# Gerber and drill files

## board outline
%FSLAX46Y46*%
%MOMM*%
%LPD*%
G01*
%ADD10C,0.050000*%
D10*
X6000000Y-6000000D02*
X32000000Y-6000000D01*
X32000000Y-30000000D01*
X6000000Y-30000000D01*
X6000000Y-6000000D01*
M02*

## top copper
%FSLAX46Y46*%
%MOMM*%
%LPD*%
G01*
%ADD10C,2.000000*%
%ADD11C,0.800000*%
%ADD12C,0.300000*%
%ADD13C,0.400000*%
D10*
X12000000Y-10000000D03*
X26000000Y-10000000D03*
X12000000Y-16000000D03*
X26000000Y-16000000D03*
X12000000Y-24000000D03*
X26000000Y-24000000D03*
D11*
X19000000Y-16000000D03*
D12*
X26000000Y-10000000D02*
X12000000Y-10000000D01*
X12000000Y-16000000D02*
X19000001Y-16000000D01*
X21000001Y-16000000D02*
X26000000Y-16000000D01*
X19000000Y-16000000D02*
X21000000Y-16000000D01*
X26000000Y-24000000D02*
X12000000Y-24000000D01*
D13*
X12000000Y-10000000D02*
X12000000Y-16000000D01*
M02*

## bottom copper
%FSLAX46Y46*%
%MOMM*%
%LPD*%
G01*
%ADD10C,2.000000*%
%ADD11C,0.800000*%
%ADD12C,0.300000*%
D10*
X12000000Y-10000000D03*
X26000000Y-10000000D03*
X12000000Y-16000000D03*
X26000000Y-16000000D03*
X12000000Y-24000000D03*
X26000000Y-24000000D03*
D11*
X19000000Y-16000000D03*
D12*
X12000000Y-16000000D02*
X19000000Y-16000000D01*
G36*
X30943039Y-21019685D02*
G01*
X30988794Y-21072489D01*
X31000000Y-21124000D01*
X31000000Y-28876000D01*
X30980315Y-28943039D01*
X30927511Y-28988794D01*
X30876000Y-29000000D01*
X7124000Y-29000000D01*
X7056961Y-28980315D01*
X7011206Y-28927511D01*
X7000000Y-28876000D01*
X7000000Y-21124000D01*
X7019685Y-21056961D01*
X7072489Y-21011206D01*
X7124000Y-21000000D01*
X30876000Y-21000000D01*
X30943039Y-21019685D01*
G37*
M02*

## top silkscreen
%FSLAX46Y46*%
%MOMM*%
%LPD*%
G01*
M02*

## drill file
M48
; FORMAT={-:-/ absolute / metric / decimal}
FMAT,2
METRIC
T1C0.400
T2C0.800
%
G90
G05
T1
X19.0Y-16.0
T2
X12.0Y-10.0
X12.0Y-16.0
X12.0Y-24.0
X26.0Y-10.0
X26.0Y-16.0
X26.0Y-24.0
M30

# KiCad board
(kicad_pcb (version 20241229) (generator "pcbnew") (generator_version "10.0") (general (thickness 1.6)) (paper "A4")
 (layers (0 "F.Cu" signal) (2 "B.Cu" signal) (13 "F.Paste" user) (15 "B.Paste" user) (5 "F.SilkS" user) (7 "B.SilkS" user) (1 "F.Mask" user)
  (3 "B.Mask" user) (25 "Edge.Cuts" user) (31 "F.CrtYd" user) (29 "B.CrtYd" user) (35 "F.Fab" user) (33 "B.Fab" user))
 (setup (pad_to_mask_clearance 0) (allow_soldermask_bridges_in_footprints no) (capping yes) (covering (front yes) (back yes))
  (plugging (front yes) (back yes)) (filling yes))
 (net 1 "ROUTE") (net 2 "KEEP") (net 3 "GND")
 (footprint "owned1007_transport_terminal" (layer "F.Cu") (at 12 10)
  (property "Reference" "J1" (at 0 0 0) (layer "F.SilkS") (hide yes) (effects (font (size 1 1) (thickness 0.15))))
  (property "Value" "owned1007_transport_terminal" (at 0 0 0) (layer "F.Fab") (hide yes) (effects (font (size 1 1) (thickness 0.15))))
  (pad "1" thru_hole circle (at 0 0) (size 2 2) (drill 0.8) (layers "*.Cu" "*.Mask") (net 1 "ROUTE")))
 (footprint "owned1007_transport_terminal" (layer "F.Cu") (at 26 10)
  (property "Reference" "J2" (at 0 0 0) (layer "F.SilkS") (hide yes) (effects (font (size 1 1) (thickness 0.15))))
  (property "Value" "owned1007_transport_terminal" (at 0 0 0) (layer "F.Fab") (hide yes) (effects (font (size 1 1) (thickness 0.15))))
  (pad "1" thru_hole circle (at 0 0) (size 2 2) (drill 0.8) (layers "*.Cu" "*.Mask") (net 1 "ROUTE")))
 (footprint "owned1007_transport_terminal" (layer "F.Cu") (at 12 16)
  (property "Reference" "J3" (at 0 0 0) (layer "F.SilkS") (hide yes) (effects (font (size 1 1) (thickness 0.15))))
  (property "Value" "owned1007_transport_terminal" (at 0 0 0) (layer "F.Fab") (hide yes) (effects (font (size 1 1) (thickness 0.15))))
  (pad "1" thru_hole circle (at 0 0) (size 2 2) (drill 0.8) (layers "*.Cu" "*.Mask") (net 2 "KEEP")))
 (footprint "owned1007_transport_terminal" (layer "F.Cu") (at 26 16)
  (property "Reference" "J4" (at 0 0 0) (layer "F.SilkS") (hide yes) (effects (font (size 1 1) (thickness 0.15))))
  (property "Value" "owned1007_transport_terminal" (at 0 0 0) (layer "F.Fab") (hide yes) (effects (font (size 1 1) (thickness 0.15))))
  (pad "1" thru_hole circle (at 0 0) (size 2 2) (drill 0.8) (layers "*.Cu" "*.Mask") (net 2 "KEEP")))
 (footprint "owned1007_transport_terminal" (layer "F.Cu") (at 12 24)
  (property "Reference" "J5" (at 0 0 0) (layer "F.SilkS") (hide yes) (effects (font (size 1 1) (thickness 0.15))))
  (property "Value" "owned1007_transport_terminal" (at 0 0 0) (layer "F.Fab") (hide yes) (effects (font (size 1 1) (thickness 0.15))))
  (pad "1" thru_hole circle (at 0 0) (size 2 2) (drill 0.8) (layers "*.Cu" "*.Mask") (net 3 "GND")))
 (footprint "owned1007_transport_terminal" (layer "F.Cu") (at 26 24)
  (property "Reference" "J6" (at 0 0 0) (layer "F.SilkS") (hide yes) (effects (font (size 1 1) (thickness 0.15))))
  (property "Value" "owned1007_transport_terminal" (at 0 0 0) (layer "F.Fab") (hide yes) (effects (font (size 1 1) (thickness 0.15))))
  (pad "1" thru_hole circle (at 0 0) (size 2 2) (drill 0.8) (layers "*.Cu" "*.Mask") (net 3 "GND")))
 (gr_rect (start 6 6) (end 32 30) (stroke (width 0.05) (type default)) (fill none) (layer "Edge.Cuts"))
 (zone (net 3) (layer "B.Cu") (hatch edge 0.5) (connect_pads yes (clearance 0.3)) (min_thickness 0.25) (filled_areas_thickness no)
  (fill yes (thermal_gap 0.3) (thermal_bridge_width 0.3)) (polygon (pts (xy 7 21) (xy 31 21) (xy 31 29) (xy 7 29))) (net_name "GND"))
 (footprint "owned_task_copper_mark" (layer "F.Cu") (at 10 28)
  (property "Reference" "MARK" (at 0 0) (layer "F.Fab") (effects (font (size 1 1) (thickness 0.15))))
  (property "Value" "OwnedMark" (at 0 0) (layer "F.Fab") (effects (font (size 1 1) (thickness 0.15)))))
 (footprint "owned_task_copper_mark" (layer "F.Cu") (at 13 28)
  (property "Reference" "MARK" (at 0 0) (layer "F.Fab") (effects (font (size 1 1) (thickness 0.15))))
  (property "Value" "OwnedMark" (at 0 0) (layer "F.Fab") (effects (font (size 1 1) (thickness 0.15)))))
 (segment (start 26 10) (end 12 10) (width 0.3) (layer "F.Cu") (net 1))
 (segment (start 12 16) (end 19.000001 16) (width 0.3) (layer "F.Cu") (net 2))
 (segment (start 21.000001 16) (end 26 16) (width 0.3) (layer "F.Cu") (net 2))
 (segment (start 19 16) (end 21 16) (width 0.3) (layer "F.Cu") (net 2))
 (via (at 19 16) (size 0.8) (drill 0.4) (layers "F.Cu" "B.Cu") (free yes) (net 2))
 (segment (start 12 16) (end 19 16) (width 0.3) (layer "B.Cu") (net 2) (locked yes))
 (segment (start 26 24) (end 12 24) (width 0.3) (layer "F.Cu") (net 3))
 (segment (start 12 10) (end 12 16) (width 0.4) (layer "F.Cu") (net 1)))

